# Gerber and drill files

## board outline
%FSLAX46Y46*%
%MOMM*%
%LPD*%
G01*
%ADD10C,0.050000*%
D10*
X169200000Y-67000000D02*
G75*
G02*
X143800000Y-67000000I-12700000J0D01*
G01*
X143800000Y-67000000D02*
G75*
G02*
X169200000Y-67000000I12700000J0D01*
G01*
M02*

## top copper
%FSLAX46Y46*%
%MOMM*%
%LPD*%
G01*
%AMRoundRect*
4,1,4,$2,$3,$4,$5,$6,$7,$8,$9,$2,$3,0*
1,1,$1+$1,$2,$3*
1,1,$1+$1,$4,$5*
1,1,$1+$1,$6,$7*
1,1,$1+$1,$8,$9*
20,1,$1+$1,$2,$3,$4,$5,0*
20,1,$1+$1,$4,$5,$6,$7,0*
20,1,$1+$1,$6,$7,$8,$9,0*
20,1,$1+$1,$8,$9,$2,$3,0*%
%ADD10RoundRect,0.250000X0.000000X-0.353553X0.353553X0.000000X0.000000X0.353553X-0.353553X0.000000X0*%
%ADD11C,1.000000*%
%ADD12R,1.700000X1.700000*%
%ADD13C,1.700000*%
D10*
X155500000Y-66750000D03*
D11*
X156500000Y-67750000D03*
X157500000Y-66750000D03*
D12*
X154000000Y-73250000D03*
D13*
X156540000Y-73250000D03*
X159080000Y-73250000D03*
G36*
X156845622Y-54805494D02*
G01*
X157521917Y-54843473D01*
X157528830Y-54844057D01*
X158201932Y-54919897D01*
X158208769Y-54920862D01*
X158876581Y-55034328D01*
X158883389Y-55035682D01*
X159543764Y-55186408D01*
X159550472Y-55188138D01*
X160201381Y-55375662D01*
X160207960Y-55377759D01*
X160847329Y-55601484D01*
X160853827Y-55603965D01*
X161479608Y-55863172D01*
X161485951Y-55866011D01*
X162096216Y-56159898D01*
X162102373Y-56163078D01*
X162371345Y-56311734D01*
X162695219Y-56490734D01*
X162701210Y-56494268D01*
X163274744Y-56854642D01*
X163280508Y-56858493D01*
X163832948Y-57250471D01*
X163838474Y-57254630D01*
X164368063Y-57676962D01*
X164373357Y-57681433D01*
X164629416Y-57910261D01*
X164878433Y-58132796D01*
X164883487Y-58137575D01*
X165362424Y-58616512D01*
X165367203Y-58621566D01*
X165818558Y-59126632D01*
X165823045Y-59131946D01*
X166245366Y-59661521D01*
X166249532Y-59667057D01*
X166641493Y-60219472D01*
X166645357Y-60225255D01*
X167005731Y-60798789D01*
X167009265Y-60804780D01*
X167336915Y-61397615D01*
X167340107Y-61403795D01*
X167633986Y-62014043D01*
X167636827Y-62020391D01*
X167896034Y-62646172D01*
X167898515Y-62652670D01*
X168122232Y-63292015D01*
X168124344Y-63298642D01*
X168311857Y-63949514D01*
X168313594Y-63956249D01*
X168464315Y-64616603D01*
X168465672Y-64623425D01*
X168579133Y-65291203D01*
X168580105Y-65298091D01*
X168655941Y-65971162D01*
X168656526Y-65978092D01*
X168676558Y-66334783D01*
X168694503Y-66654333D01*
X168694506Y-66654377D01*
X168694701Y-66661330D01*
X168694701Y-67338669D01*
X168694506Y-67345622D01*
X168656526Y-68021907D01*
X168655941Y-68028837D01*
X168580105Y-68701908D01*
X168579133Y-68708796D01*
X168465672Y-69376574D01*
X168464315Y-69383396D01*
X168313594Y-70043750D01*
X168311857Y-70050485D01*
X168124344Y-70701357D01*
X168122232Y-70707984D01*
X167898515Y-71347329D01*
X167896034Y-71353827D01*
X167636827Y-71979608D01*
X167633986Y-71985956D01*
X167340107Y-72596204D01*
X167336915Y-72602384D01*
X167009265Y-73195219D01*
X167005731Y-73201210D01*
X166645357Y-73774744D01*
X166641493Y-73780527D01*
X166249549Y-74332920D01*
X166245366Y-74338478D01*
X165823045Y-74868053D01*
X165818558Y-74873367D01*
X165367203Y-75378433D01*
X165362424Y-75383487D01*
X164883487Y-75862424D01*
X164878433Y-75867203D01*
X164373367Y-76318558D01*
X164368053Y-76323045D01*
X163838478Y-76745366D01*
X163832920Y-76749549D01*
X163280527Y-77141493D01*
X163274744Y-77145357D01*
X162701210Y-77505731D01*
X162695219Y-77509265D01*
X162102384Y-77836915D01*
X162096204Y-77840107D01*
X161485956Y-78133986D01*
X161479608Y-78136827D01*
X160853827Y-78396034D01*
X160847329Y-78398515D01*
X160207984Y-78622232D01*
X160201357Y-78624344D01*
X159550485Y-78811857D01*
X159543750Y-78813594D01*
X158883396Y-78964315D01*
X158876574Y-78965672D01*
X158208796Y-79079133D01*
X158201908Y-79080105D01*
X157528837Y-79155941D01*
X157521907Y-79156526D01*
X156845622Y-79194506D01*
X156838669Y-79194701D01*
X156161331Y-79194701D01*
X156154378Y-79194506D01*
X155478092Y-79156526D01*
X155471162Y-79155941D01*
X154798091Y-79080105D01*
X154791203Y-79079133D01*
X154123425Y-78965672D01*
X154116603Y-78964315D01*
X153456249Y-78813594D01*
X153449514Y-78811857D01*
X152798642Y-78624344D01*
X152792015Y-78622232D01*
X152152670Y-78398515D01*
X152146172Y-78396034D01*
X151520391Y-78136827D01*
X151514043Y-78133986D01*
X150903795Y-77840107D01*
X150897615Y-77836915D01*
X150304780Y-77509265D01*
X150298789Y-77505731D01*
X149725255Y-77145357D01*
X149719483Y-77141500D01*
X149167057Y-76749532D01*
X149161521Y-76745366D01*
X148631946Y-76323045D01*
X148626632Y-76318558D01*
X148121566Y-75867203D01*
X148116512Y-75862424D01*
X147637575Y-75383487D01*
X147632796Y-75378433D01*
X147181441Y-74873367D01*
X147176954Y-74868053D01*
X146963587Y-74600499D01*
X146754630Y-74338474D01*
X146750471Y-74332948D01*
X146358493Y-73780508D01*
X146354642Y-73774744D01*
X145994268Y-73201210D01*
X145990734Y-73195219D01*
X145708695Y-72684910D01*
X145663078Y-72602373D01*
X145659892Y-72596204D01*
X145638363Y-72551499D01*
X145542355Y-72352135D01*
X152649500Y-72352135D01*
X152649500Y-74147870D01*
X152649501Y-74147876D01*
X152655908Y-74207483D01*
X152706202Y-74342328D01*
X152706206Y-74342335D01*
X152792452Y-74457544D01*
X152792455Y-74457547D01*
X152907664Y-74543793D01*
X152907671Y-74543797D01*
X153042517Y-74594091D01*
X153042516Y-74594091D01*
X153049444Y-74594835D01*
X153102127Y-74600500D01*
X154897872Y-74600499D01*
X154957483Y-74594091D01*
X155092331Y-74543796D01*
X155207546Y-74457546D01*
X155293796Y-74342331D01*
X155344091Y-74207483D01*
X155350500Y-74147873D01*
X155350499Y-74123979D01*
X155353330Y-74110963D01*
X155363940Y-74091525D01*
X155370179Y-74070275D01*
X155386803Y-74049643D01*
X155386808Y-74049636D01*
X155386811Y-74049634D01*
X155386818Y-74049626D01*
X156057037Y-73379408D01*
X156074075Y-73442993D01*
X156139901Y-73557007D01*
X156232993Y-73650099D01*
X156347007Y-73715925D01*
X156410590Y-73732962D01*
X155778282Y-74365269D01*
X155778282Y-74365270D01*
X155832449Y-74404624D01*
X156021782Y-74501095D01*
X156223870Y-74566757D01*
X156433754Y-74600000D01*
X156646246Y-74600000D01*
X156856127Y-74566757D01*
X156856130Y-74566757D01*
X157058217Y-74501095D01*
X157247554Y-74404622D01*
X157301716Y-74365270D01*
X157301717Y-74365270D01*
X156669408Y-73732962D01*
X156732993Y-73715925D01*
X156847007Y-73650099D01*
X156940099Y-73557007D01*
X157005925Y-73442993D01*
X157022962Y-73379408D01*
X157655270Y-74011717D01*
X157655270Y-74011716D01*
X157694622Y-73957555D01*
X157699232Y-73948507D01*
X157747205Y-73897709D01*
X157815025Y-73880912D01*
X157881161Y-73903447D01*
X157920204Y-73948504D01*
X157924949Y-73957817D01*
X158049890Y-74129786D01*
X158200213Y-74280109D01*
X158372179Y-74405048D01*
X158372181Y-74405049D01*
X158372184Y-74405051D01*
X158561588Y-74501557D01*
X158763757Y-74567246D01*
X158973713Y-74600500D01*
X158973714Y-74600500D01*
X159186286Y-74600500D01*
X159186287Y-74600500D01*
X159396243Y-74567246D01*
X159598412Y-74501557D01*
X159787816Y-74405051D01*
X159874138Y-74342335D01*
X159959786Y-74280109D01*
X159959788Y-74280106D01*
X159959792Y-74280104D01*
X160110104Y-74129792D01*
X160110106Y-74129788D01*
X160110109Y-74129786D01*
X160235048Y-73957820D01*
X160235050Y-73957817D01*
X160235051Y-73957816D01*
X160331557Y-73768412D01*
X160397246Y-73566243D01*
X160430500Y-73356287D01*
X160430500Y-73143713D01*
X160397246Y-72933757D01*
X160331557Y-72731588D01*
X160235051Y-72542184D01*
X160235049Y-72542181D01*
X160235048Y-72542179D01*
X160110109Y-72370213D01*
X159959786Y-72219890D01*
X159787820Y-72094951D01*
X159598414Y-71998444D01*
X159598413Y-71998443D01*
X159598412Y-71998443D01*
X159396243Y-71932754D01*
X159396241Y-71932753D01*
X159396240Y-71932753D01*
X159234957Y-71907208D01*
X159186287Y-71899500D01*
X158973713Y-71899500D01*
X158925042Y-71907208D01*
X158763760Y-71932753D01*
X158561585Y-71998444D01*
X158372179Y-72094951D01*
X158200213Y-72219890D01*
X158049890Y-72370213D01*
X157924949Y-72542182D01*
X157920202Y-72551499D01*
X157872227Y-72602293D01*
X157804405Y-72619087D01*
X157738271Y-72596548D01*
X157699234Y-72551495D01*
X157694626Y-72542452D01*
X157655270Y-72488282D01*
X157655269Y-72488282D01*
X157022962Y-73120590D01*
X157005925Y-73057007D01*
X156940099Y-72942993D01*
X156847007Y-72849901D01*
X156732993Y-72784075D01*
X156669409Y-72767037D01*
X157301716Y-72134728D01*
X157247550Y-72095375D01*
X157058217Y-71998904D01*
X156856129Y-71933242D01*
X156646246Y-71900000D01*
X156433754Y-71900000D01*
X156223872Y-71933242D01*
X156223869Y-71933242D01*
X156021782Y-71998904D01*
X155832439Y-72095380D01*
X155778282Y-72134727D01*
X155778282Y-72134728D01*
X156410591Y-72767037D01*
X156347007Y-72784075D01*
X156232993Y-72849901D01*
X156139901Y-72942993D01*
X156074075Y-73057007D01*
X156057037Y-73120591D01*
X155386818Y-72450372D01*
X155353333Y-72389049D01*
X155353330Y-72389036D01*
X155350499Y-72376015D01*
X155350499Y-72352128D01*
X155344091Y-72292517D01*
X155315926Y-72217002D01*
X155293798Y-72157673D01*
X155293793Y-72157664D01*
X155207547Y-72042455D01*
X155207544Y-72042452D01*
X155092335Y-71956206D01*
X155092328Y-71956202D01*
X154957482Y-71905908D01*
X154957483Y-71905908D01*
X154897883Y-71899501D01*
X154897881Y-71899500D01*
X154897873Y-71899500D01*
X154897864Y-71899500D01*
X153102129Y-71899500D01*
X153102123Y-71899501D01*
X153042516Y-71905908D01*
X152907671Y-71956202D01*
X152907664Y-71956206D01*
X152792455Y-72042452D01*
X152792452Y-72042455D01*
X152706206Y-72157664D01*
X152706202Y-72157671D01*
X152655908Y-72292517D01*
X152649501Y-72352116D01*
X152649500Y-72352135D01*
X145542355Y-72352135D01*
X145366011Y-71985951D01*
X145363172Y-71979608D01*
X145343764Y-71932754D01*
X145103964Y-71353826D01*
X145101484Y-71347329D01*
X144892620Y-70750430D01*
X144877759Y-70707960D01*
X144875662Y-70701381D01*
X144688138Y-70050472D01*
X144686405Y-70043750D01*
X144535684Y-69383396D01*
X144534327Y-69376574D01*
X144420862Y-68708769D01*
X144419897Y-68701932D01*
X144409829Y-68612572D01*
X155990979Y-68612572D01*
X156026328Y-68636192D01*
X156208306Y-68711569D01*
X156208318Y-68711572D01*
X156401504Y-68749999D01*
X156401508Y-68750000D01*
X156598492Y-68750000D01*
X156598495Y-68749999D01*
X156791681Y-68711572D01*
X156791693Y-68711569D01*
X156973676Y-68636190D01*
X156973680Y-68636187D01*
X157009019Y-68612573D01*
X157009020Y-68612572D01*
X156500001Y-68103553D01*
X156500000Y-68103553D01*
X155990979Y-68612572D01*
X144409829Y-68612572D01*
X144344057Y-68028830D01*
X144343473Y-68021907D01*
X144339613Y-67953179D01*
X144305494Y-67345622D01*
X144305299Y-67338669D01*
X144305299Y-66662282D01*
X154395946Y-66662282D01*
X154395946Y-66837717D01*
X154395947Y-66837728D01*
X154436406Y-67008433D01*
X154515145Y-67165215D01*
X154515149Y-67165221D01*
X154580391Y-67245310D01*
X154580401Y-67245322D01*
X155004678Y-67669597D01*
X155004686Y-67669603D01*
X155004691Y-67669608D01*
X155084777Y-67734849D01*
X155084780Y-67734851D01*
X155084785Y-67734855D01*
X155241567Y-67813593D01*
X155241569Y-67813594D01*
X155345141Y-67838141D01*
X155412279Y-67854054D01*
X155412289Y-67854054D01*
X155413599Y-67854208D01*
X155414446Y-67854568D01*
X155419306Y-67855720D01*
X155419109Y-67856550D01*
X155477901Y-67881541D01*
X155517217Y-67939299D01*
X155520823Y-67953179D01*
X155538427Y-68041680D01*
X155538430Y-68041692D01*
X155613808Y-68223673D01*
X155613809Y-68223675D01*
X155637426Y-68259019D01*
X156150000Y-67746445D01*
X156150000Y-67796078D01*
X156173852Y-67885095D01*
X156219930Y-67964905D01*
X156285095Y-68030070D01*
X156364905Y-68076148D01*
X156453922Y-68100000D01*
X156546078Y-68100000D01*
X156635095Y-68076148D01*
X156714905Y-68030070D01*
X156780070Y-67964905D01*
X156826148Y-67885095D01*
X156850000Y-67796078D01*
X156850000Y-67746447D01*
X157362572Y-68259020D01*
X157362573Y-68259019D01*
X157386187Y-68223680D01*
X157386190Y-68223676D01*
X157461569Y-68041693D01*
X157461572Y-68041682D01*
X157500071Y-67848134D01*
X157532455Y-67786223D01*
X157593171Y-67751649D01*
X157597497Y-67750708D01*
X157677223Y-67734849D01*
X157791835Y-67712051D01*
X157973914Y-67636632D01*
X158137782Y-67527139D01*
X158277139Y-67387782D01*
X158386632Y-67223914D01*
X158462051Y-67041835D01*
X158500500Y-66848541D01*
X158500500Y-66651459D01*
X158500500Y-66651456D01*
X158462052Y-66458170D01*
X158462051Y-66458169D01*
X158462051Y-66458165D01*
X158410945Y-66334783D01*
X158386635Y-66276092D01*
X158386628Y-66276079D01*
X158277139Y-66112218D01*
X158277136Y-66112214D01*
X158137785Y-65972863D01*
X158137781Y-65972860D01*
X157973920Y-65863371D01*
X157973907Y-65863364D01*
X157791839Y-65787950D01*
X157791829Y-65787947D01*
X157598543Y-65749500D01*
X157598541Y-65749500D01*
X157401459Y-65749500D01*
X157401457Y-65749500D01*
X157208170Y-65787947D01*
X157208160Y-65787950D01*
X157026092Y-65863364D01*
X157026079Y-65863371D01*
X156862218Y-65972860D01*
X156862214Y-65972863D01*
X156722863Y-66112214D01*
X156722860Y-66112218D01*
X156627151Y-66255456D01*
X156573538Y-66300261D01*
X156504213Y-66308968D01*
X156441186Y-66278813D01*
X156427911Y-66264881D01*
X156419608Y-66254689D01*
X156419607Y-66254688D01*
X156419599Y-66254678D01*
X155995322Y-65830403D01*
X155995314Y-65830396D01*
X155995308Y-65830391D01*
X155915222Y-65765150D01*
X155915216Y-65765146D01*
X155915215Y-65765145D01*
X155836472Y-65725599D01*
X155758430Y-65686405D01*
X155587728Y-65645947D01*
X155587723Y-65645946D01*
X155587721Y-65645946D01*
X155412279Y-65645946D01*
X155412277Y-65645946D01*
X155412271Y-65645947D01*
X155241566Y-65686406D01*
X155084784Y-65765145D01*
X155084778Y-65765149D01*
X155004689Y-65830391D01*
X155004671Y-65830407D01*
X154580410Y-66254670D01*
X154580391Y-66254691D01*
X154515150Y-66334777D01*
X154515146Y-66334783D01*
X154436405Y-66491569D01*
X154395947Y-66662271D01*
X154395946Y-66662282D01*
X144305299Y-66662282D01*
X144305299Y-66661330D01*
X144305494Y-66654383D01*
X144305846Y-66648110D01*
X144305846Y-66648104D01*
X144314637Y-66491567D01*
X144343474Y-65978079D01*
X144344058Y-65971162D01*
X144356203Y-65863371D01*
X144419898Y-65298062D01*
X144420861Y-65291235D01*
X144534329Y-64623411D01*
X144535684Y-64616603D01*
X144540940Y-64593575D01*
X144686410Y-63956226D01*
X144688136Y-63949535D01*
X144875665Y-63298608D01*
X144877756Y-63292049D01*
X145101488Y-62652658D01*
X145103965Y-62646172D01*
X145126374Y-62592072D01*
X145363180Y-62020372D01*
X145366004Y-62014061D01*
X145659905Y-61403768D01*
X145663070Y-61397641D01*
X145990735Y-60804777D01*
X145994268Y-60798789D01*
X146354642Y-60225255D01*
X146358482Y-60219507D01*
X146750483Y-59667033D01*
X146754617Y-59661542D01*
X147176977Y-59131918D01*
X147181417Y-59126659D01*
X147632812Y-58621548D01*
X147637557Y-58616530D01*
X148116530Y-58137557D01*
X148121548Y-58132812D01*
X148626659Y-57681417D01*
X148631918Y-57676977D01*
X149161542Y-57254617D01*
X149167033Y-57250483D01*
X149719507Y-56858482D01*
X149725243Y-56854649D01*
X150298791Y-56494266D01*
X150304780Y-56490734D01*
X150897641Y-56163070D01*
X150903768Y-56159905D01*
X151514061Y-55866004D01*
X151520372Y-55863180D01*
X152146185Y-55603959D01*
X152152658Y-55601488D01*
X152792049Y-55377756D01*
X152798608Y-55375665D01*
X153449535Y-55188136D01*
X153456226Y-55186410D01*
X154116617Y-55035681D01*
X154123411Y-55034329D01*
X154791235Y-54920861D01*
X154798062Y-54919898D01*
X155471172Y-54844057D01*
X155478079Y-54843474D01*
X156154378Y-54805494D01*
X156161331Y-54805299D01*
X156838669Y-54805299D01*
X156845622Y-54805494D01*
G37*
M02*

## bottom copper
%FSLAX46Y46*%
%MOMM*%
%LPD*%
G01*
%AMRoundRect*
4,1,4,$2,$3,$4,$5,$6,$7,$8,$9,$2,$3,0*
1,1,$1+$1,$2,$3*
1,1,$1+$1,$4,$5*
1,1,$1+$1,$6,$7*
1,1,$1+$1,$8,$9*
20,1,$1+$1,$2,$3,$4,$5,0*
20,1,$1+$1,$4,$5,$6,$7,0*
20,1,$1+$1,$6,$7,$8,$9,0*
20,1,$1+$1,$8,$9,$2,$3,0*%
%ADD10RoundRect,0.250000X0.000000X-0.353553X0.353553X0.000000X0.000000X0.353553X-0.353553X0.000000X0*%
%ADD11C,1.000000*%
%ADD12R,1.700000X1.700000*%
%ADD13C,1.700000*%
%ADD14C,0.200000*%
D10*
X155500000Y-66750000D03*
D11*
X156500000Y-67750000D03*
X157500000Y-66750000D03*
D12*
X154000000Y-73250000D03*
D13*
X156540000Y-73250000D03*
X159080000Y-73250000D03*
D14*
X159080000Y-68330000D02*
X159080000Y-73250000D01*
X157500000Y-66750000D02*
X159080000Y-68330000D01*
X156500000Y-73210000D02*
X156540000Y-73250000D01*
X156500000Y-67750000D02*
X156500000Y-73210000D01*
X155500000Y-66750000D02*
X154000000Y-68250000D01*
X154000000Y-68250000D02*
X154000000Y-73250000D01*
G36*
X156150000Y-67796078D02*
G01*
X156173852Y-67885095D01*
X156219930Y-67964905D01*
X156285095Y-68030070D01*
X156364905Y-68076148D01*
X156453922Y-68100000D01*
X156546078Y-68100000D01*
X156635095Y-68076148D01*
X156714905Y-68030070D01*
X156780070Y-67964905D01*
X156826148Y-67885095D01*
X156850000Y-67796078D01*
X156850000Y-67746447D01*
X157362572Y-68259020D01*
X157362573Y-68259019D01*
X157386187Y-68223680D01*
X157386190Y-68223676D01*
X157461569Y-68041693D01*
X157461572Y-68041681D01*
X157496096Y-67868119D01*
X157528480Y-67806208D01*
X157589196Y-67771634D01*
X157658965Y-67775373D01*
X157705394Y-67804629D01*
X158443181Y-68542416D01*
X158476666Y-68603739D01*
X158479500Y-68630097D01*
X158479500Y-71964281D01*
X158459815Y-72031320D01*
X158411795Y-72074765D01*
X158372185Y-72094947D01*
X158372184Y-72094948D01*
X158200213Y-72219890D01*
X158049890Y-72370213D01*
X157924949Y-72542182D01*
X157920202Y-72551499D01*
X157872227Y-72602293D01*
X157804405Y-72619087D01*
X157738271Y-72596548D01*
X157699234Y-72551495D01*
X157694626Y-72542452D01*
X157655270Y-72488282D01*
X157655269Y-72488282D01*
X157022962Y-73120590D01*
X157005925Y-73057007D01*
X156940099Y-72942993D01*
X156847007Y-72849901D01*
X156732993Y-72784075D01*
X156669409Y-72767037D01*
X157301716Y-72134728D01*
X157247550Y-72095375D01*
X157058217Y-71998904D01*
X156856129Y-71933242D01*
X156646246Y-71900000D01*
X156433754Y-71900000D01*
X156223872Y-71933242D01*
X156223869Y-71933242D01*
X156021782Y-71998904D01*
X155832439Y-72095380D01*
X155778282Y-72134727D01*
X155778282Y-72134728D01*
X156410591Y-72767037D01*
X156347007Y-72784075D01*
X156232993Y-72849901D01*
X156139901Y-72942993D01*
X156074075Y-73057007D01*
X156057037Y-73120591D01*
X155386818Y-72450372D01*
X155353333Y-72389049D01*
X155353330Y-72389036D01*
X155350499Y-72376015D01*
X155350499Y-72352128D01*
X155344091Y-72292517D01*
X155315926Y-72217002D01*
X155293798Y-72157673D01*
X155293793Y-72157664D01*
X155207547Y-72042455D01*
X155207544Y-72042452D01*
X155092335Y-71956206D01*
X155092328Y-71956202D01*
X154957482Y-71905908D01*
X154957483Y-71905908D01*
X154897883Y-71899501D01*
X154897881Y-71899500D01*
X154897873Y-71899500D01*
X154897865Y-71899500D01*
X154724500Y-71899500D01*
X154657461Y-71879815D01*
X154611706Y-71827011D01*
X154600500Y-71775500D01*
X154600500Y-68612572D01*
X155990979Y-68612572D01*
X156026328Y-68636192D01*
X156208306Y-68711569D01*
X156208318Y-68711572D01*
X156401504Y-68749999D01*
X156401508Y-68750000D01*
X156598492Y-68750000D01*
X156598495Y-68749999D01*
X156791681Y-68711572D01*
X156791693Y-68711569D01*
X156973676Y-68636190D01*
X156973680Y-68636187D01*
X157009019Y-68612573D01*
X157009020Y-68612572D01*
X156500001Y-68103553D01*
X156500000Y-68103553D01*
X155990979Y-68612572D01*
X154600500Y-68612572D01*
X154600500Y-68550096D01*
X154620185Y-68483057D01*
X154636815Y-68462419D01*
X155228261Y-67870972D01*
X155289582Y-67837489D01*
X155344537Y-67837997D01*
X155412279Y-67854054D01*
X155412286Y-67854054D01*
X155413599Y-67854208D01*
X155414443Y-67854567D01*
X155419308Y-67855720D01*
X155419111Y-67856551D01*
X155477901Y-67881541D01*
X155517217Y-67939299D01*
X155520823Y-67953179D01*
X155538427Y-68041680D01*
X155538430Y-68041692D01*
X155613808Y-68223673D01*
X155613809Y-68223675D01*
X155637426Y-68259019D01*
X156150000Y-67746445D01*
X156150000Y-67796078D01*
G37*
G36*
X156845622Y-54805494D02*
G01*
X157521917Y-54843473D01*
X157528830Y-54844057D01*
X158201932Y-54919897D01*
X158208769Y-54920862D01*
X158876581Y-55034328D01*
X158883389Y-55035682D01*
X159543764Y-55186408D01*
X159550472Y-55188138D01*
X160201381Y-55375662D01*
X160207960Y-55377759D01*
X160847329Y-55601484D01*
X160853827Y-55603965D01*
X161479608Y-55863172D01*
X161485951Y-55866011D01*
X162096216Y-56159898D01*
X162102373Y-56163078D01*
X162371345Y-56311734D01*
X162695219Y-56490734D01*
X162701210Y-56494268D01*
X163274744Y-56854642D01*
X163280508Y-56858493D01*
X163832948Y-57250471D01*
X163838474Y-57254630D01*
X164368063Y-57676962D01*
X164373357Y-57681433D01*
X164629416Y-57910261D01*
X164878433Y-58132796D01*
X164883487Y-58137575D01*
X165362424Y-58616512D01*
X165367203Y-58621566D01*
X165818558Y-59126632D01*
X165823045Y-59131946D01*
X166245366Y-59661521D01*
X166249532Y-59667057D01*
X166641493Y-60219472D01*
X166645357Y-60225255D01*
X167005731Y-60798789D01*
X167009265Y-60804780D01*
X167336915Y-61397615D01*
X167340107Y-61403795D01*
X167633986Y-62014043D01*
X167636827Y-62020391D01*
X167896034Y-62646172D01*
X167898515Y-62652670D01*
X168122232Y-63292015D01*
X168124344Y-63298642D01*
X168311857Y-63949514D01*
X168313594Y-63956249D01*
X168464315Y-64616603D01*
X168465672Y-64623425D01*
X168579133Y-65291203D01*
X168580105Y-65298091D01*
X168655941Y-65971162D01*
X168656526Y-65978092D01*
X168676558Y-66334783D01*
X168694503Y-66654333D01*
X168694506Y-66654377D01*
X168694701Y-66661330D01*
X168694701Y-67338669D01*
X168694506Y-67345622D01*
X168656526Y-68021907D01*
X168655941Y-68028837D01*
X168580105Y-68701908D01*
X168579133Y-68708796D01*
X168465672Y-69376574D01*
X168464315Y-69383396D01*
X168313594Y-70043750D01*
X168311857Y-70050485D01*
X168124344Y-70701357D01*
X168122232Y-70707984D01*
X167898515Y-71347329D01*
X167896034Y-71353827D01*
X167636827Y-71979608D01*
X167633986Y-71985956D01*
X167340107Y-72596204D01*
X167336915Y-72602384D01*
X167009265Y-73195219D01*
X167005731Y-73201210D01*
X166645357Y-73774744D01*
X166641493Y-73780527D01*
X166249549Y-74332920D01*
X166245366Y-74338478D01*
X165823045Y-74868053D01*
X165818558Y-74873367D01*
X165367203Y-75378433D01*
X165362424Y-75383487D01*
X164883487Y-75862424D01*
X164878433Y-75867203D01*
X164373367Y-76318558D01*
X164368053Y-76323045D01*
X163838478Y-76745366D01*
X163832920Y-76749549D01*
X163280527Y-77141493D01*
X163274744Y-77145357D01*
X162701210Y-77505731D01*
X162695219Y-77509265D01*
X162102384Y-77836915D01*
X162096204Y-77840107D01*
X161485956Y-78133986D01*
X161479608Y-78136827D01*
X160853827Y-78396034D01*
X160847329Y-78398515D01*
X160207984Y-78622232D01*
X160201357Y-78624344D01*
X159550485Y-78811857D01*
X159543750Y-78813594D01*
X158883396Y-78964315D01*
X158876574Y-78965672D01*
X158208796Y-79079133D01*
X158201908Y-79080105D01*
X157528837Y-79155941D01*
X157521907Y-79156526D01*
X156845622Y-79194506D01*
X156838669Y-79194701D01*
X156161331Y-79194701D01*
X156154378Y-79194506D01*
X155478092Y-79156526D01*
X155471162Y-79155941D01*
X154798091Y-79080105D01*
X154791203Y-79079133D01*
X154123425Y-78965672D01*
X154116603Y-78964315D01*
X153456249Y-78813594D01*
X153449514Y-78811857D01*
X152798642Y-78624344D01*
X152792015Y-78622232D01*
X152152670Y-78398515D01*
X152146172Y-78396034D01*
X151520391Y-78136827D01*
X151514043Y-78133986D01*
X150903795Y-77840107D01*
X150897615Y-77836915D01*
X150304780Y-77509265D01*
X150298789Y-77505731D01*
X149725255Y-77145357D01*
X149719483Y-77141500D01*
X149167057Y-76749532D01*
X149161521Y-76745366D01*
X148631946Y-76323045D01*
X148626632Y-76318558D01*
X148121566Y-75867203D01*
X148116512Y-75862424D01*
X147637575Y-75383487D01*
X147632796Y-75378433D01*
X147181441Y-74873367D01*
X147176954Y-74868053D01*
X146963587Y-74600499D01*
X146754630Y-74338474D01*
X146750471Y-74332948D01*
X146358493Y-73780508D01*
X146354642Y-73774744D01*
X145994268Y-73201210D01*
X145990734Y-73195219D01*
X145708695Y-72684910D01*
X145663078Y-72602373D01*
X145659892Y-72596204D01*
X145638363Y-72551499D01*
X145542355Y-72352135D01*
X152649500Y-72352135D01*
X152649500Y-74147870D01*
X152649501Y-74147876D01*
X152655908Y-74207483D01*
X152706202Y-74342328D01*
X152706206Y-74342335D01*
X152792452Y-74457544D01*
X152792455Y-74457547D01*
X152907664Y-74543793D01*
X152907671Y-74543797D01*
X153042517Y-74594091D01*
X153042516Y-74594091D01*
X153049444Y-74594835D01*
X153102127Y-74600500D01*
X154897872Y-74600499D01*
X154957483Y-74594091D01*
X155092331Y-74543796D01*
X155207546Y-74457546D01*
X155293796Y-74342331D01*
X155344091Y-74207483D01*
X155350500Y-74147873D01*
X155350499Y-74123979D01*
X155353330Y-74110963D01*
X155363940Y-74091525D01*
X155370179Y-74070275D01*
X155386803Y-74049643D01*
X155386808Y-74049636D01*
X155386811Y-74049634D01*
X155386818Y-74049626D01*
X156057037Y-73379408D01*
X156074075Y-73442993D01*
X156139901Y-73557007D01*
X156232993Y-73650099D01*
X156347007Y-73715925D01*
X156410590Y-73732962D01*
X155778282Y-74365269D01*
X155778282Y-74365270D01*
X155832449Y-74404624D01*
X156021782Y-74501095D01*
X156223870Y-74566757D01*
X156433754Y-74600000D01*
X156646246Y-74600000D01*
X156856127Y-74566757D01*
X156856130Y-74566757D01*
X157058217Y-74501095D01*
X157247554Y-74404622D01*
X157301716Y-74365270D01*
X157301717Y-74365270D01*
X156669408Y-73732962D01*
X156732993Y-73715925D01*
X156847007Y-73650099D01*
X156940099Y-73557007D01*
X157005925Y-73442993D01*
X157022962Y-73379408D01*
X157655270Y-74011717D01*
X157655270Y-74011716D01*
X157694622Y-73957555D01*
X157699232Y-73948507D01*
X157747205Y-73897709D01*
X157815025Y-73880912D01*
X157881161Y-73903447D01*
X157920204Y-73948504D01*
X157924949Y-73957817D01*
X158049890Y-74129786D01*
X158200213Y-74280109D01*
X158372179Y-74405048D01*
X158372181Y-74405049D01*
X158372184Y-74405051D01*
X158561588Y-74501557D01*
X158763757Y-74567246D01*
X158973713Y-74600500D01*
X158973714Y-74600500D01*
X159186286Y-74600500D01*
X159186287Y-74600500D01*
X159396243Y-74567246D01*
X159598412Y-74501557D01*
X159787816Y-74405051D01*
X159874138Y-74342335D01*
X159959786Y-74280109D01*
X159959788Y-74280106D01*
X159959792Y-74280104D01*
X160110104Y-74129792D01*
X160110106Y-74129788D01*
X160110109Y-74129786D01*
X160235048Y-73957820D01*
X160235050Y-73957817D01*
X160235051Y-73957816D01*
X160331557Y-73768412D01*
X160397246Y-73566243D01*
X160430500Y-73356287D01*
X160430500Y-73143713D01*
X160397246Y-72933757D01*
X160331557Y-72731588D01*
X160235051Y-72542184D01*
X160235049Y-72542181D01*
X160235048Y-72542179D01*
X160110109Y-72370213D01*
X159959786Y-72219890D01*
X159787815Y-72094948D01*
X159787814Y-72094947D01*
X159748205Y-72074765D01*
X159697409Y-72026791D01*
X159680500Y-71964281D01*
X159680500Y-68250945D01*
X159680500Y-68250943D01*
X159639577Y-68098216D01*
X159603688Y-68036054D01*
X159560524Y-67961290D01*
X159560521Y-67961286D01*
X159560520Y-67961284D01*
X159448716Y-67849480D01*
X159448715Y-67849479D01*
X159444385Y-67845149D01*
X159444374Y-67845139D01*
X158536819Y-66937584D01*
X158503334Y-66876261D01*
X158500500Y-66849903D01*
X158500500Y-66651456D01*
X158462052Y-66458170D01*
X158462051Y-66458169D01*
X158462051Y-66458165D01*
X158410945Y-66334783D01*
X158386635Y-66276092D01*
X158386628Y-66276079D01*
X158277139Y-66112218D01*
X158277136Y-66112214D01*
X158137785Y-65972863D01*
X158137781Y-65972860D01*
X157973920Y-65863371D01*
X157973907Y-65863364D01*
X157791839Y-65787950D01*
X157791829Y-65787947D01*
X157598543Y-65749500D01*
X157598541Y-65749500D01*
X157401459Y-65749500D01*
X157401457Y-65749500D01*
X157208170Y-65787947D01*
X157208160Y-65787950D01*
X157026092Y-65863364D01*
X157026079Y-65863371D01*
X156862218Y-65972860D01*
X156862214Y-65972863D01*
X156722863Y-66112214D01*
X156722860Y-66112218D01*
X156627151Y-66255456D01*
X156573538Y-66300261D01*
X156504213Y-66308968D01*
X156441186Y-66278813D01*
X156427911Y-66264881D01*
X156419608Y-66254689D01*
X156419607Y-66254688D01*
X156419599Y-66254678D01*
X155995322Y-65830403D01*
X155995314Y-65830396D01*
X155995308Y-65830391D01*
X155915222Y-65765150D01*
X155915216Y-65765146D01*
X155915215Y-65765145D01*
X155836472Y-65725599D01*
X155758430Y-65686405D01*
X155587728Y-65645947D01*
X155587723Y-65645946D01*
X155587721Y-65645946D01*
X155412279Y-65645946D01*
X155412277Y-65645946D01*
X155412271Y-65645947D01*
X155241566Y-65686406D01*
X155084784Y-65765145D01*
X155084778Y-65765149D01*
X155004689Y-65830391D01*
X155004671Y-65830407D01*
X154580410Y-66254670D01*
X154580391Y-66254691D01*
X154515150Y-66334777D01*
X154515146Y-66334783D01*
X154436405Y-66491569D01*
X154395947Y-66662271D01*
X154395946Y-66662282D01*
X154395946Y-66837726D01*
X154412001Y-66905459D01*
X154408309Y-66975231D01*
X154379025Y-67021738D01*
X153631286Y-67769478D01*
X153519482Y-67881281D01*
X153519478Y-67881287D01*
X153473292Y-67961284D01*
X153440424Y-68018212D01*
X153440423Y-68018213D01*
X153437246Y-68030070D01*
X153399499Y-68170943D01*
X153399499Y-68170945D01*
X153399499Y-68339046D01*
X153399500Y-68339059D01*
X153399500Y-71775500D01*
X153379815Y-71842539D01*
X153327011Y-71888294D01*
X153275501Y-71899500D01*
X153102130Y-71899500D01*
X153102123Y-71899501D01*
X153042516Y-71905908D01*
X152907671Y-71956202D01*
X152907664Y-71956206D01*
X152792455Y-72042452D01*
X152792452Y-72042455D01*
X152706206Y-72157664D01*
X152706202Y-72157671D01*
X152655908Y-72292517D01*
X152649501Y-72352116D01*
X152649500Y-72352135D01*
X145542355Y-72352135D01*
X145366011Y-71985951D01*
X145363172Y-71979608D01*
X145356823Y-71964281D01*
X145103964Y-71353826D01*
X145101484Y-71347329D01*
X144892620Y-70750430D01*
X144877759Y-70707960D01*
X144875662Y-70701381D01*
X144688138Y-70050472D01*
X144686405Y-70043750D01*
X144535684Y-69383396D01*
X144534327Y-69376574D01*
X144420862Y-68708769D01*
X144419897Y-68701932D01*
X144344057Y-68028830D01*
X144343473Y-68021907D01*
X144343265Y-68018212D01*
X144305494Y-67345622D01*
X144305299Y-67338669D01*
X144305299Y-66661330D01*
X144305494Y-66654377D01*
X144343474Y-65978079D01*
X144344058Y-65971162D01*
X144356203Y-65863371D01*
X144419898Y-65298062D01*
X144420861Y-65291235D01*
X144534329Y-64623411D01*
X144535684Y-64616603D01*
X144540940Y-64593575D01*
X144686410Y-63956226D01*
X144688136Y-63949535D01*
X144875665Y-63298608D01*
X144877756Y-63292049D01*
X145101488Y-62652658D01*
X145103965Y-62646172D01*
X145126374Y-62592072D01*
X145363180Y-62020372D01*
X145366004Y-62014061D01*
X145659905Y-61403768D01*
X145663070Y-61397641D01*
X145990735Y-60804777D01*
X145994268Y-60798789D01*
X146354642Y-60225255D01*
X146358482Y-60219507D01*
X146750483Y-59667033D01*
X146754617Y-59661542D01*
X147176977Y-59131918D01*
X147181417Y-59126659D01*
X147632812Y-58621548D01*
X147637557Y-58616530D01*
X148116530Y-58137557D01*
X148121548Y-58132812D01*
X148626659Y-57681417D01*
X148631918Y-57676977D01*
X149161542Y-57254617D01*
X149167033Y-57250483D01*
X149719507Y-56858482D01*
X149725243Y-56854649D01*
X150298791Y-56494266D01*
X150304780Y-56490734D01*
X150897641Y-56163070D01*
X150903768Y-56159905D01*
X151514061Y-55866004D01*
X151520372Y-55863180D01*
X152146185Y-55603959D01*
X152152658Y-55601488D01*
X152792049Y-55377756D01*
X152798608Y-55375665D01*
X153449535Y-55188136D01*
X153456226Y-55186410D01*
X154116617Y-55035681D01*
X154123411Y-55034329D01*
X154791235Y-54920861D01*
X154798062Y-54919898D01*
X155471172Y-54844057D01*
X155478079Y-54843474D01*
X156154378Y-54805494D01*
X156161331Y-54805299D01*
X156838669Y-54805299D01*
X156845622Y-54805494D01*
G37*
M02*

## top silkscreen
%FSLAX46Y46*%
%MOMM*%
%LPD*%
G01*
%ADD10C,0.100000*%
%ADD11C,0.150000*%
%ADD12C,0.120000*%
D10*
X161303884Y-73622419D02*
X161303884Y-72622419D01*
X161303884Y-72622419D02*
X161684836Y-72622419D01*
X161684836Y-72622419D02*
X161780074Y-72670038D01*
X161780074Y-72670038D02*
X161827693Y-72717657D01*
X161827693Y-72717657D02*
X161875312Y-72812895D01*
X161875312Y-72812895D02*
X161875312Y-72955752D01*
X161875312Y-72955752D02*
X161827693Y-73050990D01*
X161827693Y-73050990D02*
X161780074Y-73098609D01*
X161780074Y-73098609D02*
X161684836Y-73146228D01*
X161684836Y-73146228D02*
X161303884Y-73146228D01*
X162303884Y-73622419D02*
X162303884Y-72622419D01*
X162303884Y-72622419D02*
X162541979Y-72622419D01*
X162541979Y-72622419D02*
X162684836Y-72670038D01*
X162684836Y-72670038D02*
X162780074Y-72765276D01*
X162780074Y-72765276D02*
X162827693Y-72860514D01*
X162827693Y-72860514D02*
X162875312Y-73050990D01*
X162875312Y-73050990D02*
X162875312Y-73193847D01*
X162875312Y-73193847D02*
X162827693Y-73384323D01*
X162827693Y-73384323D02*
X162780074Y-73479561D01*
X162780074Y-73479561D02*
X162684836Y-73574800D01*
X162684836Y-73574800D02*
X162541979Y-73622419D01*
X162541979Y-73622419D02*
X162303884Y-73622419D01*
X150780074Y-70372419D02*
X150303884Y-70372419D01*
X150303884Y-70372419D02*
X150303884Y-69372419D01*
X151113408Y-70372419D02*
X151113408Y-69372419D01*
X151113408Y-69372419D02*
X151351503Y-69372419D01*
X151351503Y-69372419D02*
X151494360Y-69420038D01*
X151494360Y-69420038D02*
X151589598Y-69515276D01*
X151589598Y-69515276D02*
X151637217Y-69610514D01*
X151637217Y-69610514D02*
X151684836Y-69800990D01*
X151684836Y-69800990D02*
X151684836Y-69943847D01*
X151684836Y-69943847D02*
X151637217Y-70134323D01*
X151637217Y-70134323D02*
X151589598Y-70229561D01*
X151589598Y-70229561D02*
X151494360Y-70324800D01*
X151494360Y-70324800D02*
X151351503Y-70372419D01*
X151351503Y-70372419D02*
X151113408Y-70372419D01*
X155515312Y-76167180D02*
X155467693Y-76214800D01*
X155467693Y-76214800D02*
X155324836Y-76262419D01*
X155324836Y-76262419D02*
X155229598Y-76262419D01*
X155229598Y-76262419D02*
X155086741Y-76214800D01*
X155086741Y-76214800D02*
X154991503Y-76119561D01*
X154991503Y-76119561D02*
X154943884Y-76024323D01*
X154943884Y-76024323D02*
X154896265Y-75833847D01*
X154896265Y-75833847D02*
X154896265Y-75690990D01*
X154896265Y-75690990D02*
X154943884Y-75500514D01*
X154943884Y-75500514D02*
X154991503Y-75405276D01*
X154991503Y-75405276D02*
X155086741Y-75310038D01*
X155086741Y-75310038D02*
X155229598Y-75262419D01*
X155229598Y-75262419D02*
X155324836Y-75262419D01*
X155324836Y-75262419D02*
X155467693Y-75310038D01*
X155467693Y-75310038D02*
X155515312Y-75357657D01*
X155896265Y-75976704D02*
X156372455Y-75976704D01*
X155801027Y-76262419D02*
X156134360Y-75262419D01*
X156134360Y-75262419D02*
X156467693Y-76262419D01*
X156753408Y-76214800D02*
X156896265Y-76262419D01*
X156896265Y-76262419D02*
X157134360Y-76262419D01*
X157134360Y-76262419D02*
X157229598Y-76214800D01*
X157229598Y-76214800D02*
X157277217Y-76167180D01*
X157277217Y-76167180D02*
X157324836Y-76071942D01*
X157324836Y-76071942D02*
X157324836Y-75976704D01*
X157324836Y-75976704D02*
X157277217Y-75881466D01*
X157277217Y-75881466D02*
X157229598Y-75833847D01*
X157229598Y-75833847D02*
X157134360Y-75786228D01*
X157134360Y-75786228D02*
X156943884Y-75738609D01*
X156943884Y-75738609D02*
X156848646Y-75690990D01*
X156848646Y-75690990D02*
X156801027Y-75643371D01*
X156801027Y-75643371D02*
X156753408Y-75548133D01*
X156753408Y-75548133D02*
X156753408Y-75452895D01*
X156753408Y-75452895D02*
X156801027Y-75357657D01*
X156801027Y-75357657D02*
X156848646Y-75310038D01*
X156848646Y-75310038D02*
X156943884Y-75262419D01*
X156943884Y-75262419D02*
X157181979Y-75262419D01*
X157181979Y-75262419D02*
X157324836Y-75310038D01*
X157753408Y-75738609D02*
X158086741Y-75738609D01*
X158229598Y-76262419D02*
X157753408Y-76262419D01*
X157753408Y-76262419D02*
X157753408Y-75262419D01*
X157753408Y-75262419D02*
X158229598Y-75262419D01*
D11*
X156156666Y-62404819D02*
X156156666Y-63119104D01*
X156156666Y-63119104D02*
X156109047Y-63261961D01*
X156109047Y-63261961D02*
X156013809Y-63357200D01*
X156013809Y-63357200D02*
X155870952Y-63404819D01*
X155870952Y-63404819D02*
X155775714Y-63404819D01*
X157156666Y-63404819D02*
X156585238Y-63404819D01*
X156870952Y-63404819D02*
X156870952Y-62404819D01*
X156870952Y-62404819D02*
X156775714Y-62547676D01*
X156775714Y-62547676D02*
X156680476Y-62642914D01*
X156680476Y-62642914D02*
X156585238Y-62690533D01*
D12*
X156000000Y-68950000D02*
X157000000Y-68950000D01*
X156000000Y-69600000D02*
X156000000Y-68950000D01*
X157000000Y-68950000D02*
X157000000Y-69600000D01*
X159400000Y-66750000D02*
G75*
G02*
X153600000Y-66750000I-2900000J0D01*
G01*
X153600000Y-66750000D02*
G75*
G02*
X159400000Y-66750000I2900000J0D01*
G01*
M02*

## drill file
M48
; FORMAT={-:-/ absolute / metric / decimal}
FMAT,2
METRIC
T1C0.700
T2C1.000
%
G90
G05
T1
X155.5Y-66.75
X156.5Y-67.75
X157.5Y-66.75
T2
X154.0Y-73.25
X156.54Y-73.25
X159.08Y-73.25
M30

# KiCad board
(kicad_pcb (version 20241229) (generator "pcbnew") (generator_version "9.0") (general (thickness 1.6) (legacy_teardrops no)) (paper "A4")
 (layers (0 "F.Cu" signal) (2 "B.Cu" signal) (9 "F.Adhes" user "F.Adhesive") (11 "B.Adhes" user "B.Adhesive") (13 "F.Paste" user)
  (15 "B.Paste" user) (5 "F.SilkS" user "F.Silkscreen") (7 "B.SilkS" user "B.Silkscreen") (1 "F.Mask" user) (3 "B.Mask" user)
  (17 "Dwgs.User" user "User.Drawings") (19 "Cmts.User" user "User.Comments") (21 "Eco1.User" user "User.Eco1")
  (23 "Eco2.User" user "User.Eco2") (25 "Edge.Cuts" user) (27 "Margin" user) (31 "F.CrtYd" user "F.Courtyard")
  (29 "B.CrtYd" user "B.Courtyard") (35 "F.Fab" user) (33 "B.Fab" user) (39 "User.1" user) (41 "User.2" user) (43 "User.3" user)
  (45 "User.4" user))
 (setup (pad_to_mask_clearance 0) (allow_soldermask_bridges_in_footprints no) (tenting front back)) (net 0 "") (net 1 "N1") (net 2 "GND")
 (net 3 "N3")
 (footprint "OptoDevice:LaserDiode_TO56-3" (layer "F.Cu") (at 155.5 66.75)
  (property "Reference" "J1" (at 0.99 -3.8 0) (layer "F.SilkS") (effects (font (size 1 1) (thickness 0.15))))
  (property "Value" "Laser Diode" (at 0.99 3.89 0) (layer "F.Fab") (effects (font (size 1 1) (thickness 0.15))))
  (fp_line (start 0.5 2.2) (end 1.5 2.2) (stroke (width 0.12) (type solid)) (layer "F.SilkS"))
  (fp_line (start 0.5 2.85) (end 0.5 2.2) (stroke (width 0.12) (type solid)) (layer "F.SilkS"))
  (fp_line (start 1.5 2.2) (end 1.5 2.85) (stroke (width 0.12) (type solid)) (layer "F.SilkS"))
  (fp_circle (center 1 0) (end 3.9 0) (stroke (width 0.12) (type solid)) (fill no) (layer "F.SilkS"))
  (pad "1" thru_hole roundrect (at 0 0 45) (size 1 1) (drill 0.7) (layers "*.Cu" "*.Mask") (remove_unused_layers no) (roundrect_rratio 0.25)
   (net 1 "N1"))
  (pad "2" thru_hole circle (at 1 1) (size 1 1) (drill 0.7) (layers "*.Cu" "*.Mask") (remove_unused_layers no) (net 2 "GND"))
  (pad "3" thru_hole circle (at 2 0) (size 1 1) (drill 0.7) (layers "*.Cu" "*.Mask") (remove_unused_layers no) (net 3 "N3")))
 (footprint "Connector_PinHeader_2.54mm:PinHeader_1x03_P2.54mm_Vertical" (layer "B.Cu") (at 154 73.25 -90)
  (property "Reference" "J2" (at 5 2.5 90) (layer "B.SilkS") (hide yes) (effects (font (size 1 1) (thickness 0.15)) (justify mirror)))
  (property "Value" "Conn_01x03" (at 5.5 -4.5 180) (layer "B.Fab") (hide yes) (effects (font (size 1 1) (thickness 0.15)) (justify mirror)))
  (pad "1" thru_hole rect (at 0 0 270) (size 1.7 1.7) (drill 1) (layers "*.Cu" "*.Mask") (remove_unused_layers no) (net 1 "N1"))
  (pad "2" thru_hole circle (at 0 -2.54 270) (size 1.7 1.7) (drill 1) (layers "*.Cu" "*.Mask") (remove_unused_layers no) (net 2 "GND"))
  (pad "3" thru_hole circle (at 0 -5.08 270) (size 1.7 1.7) (drill 1) (layers "*.Cu" "*.Mask") (remove_unused_layers no) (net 3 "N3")))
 (gr_circle (center 156.5 67) (end 169.2 67) (stroke (width 0.05) (type solid)) (fill no) (layer "Edge.Cuts"))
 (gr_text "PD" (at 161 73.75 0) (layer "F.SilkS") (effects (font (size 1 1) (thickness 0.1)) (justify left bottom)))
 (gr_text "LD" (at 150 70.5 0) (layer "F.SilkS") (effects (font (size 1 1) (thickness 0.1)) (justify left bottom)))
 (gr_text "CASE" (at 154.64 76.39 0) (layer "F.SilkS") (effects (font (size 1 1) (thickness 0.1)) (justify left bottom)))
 (segment (start 159.08 68.33) (end 159.08 73.25) (width 0.2) (layer "B.Cu") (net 3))
 (segment (start 157.5 66.75) (end 159.08 68.33) (width 0.2) (layer "B.Cu") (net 3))
 (segment (start 156.5 73.21) (end 156.54 73.25) (width 0.2) (layer "B.Cu") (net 2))
 (segment (start 156.5 67.75) (end 156.5 73.21) (width 0.2) (layer "B.Cu") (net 2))
 (segment (start 155.5 66.75) (end 154 68.25) (width 0.2) (layer "B.Cu") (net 1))
 (segment (start 154 68.25) (end 154 73.25) (width 0.2) (layer "B.Cu") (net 1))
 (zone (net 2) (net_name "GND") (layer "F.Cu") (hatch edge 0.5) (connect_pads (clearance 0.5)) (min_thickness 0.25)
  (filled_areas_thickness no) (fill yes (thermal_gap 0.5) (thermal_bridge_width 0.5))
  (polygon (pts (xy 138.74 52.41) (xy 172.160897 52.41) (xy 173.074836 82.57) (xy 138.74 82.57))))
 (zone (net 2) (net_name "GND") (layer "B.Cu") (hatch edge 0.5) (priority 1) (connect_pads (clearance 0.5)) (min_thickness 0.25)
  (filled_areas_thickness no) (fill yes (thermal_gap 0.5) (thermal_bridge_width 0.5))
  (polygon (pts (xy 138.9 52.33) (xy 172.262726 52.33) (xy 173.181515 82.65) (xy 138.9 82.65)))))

